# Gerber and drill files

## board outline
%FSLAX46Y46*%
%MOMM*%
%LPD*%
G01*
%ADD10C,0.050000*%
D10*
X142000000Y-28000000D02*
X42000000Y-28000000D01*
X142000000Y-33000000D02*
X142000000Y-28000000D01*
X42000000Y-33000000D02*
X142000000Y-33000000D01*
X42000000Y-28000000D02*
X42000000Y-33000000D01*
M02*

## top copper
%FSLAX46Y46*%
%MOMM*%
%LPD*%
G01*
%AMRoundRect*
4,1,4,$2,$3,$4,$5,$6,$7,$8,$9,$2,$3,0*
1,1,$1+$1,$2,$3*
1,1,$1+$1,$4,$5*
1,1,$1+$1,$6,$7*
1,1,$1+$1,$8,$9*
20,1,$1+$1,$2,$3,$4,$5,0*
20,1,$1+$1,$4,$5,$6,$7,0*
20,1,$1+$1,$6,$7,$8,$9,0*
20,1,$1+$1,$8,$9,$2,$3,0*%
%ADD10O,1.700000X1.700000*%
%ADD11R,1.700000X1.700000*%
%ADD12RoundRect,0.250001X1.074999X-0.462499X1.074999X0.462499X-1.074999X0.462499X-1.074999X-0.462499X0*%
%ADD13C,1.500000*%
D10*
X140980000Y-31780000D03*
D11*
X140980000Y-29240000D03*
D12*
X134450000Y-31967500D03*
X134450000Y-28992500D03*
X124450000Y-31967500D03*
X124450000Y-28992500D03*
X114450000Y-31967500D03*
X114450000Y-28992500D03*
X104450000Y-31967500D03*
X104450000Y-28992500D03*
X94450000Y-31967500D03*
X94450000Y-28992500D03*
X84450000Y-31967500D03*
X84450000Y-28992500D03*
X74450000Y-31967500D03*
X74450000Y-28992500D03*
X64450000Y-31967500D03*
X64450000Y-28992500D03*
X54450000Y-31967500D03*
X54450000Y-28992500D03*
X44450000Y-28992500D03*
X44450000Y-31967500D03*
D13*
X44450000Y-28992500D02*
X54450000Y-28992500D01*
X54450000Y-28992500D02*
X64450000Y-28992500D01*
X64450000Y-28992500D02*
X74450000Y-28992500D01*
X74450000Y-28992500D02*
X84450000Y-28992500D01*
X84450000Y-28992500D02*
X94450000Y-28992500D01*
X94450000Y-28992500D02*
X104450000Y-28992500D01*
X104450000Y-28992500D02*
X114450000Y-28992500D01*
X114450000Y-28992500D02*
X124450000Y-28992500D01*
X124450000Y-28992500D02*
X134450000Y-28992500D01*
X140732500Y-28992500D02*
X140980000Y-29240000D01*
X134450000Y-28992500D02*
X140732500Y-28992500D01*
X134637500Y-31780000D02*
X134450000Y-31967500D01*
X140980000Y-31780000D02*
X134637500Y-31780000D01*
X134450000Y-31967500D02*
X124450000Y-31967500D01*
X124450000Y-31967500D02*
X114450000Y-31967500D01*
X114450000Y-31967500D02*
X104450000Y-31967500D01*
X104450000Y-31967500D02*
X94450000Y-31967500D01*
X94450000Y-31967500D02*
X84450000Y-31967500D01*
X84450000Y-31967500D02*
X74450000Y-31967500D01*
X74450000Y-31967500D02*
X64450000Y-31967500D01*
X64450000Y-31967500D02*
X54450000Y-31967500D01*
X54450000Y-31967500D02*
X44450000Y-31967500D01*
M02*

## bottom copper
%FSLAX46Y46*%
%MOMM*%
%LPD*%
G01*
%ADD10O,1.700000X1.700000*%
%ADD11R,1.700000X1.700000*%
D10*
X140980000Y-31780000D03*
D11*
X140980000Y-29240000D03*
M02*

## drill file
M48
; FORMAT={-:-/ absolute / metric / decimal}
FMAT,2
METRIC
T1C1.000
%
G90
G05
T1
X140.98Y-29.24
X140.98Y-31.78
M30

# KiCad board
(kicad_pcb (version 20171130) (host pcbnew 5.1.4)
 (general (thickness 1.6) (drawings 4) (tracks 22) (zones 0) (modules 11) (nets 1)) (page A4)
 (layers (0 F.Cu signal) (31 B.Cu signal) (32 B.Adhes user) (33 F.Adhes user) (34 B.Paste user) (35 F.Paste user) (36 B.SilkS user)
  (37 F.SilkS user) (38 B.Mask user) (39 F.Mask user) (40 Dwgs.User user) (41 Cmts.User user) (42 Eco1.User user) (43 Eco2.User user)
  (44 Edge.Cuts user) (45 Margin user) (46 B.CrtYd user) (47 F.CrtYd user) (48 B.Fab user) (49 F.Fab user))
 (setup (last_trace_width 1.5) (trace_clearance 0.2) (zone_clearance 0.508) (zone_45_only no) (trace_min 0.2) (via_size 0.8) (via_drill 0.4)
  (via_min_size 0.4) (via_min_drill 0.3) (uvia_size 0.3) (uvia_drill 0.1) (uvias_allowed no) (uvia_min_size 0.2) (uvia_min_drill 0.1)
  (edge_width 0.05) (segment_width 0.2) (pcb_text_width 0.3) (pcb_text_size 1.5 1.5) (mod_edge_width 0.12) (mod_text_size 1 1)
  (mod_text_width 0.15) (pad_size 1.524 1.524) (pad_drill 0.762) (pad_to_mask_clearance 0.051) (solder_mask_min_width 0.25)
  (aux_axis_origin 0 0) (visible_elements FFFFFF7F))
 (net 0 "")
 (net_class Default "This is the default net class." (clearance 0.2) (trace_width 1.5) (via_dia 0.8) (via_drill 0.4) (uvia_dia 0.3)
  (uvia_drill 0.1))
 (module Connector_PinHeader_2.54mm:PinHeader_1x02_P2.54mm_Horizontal (layer F.Cu) (at 140.98 29.24)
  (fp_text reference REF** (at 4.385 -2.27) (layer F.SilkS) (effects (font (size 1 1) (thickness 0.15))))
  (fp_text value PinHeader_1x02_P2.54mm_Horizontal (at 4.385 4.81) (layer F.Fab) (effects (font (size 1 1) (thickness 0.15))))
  (pad 2 thru_hole oval (at 0 2.54) (size 1.7 1.7) (drill 1) (layers *.Cu *.Mask))
  (pad 1 thru_hole rect (at 0 0) (size 1.7 1.7) (drill 1) (layers *.Cu *.Mask)))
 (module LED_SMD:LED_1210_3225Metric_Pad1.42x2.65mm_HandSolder (layer F.Cu) (at 134.45 30.48 90)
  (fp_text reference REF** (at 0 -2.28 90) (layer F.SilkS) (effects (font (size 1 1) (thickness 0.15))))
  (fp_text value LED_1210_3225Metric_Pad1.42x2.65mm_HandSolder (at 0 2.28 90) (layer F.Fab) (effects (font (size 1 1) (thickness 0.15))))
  (pad 1 smd roundrect (at -1.4875 0 90) (size 1.425 2.65) (layers F.Cu F.Paste F.Mask) (roundrect_rratio 0.175439))
  (pad 2 smd roundrect (at 1.4875 0 90) (size 1.425 2.65) (layers F.Cu F.Paste F.Mask) (roundrect_rratio 0.175439)))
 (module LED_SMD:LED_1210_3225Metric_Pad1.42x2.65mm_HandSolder (layer F.Cu) (at 124.45 30.48 90)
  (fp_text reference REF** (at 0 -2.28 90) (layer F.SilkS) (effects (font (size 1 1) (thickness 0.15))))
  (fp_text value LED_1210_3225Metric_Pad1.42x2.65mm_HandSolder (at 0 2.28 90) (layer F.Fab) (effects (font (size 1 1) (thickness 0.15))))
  (pad 1 smd roundrect (at -1.4875 0 90) (size 1.425 2.65) (layers F.Cu F.Paste F.Mask) (roundrect_rratio 0.175439))
  (pad 2 smd roundrect (at 1.4875 0 90) (size 1.425 2.65) (layers F.Cu F.Paste F.Mask) (roundrect_rratio 0.175439)))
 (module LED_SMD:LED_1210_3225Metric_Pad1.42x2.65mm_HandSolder (layer F.Cu) (at 114.45 30.48 90)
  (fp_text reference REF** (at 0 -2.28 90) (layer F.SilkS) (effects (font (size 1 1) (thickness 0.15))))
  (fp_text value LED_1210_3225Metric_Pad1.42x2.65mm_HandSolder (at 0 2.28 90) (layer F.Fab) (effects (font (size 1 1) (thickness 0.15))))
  (pad 1 smd roundrect (at -1.4875 0 90) (size 1.425 2.65) (layers F.Cu F.Paste F.Mask) (roundrect_rratio 0.175439))
  (pad 2 smd roundrect (at 1.4875 0 90) (size 1.425 2.65) (layers F.Cu F.Paste F.Mask) (roundrect_rratio 0.175439)))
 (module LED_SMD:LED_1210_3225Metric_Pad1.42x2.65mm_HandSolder (layer F.Cu) (at 104.45 30.48 90)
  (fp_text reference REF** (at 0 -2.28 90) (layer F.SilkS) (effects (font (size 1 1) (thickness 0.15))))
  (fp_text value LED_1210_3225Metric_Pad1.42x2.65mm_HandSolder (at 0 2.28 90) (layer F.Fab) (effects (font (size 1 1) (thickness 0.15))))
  (pad 1 smd roundrect (at -1.4875 0 90) (size 1.425 2.65) (layers F.Cu F.Paste F.Mask) (roundrect_rratio 0.175439))
  (pad 2 smd roundrect (at 1.4875 0 90) (size 1.425 2.65) (layers F.Cu F.Paste F.Mask) (roundrect_rratio 0.175439)))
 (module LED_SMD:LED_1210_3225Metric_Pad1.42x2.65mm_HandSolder (layer F.Cu) (at 94.45 30.48 90)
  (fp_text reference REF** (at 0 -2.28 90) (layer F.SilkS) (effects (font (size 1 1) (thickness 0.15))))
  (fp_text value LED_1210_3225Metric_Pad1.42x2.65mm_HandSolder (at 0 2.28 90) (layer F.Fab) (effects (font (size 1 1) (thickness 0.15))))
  (pad 1 smd roundrect (at -1.4875 0 90) (size 1.425 2.65) (layers F.Cu F.Paste F.Mask) (roundrect_rratio 0.175439))
  (pad 2 smd roundrect (at 1.4875 0 90) (size 1.425 2.65) (layers F.Cu F.Paste F.Mask) (roundrect_rratio 0.175439)))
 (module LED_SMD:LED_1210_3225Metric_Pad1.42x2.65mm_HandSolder (layer F.Cu) (at 84.45 30.48 90)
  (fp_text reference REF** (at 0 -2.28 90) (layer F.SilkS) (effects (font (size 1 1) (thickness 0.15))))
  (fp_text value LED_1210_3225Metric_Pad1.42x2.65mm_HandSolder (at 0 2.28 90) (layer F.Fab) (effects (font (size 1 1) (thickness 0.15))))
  (pad 1 smd roundrect (at -1.4875 0 90) (size 1.425 2.65) (layers F.Cu F.Paste F.Mask) (roundrect_rratio 0.175439))
  (pad 2 smd roundrect (at 1.4875 0 90) (size 1.425 2.65) (layers F.Cu F.Paste F.Mask) (roundrect_rratio 0.175439)))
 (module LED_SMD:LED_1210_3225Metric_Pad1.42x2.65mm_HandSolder (layer F.Cu) (at 74.45 30.48 90)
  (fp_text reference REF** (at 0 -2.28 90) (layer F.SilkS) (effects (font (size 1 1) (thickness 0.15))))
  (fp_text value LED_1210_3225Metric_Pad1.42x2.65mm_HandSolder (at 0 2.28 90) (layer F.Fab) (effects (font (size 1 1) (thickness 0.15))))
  (pad 1 smd roundrect (at -1.4875 0 90) (size 1.425 2.65) (layers F.Cu F.Paste F.Mask) (roundrect_rratio 0.175439))
  (pad 2 smd roundrect (at 1.4875 0 90) (size 1.425 2.65) (layers F.Cu F.Paste F.Mask) (roundrect_rratio 0.175439)))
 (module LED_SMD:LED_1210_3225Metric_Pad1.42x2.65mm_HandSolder (layer F.Cu) (at 64.45 30.48 90)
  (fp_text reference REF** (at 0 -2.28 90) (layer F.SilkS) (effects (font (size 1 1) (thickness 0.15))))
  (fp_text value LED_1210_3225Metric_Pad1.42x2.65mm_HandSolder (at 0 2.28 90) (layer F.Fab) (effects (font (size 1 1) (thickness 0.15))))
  (pad 1 smd roundrect (at -1.4875 0 90) (size 1.425 2.65) (layers F.Cu F.Paste F.Mask) (roundrect_rratio 0.175439))
  (pad 2 smd roundrect (at 1.4875 0 90) (size 1.425 2.65) (layers F.Cu F.Paste F.Mask) (roundrect_rratio 0.175439)))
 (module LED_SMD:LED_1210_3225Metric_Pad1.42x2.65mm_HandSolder (layer F.Cu) (at 54.45 30.48 90)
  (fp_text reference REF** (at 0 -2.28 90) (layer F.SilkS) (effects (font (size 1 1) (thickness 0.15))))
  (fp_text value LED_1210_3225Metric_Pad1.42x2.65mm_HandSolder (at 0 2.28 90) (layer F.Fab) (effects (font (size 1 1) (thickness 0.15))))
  (pad 1 smd roundrect (at -1.4875 0 90) (size 1.425 2.65) (layers F.Cu F.Paste F.Mask) (roundrect_rratio 0.175439))
  (pad 2 smd roundrect (at 1.4875 0 90) (size 1.425 2.65) (layers F.Cu F.Paste F.Mask) (roundrect_rratio 0.175439)))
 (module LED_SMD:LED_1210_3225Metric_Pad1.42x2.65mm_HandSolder (layer F.Cu) (at 44.45 30.48 90)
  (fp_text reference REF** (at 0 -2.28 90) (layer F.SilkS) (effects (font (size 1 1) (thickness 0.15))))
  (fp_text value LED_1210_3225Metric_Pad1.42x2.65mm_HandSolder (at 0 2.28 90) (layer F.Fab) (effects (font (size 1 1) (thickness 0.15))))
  (pad 2 smd roundrect (at 1.4875 0 90) (size 1.425 2.65) (layers F.Cu F.Paste F.Mask) (roundrect_rratio 0.175439))
  (pad 1 smd roundrect (at -1.4875 0 90) (size 1.425 2.65) (layers F.Cu F.Paste F.Mask) (roundrect_rratio 0.175439)))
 (gr_line (start 142 28) (end 42 28) (layer Edge.Cuts) (width 0.05))
 (gr_line (start 142 33) (end 142 28) (layer Edge.Cuts) (width 0.05))
 (gr_line (start 42 33) (end 142 33) (layer Edge.Cuts) (width 0.05))
 (gr_line (start 42 28) (end 42 33) (layer Edge.Cuts) (width 0.05))
 (segment (start 44.45 28.9925) (end 54.45 28.9925) (width 1.5) (layer F.Cu) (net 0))
 (segment (start 54.45 28.9925) (end 64.45 28.9925) (width 1.5) (layer F.Cu) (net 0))
 (segment (start 64.45 28.9925) (end 74.45 28.9925) (width 1.5) (layer F.Cu) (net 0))
 (segment (start 74.45 28.9925) (end 84.45 28.9925) (width 1.5) (layer F.Cu) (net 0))
 (segment (start 84.45 28.9925) (end 94.45 28.9925) (width 1.5) (layer F.Cu) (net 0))
 (segment (start 94.45 28.9925) (end 104.45 28.9925) (width 1.5) (layer F.Cu) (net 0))
 (segment (start 104.45 28.9925) (end 114.45 28.9925) (width 1.5) (layer F.Cu) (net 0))
 (segment (start 114.45 28.9925) (end 124.45 28.9925) (width 1.5) (layer F.Cu) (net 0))
 (segment (start 124.45 28.9925) (end 134.45 28.9925) (width 1.5) (layer F.Cu) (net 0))
 (segment (start 140.7325 28.9925) (end 140.98 29.24) (width 1.5) (layer F.Cu) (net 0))
 (segment (start 134.45 28.9925) (end 140.7325 28.9925) (width 1.5) (layer F.Cu) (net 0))
 (segment (start 134.6375 31.78) (end 134.45 31.9675) (width 1.5) (layer F.Cu) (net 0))
 (segment (start 140.98 31.78) (end 134.6375 31.78) (width 1.5) (layer F.Cu) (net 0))
 (segment (start 134.45 31.9675) (end 124.45 31.9675) (width 1.5) (layer F.Cu) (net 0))
 (segment (start 124.45 31.9675) (end 114.45 31.9675) (width 1.5) (layer F.Cu) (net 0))
 (segment (start 114.45 31.9675) (end 104.45 31.9675) (width 1.5) (layer F.Cu) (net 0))
 (segment (start 104.45 31.9675) (end 94.45 31.9675) (width 1.5) (layer F.Cu) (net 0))
 (segment (start 94.45 31.9675) (end 84.45 31.9675) (width 1.5) (layer F.Cu) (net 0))
 (segment (start 84.45 31.9675) (end 74.45 31.9675) (width 1.5) (layer F.Cu) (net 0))
 (segment (start 74.45 31.9675) (end 64.45 31.9675) (width 1.5) (layer F.Cu) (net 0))
 (segment (start 64.45 31.9675) (end 54.45 31.9675) (width 1.5) (layer F.Cu) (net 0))
 (segment (start 54.45 31.9675) (end 44.45 31.9675) (width 1.5) (layer F.Cu) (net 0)))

